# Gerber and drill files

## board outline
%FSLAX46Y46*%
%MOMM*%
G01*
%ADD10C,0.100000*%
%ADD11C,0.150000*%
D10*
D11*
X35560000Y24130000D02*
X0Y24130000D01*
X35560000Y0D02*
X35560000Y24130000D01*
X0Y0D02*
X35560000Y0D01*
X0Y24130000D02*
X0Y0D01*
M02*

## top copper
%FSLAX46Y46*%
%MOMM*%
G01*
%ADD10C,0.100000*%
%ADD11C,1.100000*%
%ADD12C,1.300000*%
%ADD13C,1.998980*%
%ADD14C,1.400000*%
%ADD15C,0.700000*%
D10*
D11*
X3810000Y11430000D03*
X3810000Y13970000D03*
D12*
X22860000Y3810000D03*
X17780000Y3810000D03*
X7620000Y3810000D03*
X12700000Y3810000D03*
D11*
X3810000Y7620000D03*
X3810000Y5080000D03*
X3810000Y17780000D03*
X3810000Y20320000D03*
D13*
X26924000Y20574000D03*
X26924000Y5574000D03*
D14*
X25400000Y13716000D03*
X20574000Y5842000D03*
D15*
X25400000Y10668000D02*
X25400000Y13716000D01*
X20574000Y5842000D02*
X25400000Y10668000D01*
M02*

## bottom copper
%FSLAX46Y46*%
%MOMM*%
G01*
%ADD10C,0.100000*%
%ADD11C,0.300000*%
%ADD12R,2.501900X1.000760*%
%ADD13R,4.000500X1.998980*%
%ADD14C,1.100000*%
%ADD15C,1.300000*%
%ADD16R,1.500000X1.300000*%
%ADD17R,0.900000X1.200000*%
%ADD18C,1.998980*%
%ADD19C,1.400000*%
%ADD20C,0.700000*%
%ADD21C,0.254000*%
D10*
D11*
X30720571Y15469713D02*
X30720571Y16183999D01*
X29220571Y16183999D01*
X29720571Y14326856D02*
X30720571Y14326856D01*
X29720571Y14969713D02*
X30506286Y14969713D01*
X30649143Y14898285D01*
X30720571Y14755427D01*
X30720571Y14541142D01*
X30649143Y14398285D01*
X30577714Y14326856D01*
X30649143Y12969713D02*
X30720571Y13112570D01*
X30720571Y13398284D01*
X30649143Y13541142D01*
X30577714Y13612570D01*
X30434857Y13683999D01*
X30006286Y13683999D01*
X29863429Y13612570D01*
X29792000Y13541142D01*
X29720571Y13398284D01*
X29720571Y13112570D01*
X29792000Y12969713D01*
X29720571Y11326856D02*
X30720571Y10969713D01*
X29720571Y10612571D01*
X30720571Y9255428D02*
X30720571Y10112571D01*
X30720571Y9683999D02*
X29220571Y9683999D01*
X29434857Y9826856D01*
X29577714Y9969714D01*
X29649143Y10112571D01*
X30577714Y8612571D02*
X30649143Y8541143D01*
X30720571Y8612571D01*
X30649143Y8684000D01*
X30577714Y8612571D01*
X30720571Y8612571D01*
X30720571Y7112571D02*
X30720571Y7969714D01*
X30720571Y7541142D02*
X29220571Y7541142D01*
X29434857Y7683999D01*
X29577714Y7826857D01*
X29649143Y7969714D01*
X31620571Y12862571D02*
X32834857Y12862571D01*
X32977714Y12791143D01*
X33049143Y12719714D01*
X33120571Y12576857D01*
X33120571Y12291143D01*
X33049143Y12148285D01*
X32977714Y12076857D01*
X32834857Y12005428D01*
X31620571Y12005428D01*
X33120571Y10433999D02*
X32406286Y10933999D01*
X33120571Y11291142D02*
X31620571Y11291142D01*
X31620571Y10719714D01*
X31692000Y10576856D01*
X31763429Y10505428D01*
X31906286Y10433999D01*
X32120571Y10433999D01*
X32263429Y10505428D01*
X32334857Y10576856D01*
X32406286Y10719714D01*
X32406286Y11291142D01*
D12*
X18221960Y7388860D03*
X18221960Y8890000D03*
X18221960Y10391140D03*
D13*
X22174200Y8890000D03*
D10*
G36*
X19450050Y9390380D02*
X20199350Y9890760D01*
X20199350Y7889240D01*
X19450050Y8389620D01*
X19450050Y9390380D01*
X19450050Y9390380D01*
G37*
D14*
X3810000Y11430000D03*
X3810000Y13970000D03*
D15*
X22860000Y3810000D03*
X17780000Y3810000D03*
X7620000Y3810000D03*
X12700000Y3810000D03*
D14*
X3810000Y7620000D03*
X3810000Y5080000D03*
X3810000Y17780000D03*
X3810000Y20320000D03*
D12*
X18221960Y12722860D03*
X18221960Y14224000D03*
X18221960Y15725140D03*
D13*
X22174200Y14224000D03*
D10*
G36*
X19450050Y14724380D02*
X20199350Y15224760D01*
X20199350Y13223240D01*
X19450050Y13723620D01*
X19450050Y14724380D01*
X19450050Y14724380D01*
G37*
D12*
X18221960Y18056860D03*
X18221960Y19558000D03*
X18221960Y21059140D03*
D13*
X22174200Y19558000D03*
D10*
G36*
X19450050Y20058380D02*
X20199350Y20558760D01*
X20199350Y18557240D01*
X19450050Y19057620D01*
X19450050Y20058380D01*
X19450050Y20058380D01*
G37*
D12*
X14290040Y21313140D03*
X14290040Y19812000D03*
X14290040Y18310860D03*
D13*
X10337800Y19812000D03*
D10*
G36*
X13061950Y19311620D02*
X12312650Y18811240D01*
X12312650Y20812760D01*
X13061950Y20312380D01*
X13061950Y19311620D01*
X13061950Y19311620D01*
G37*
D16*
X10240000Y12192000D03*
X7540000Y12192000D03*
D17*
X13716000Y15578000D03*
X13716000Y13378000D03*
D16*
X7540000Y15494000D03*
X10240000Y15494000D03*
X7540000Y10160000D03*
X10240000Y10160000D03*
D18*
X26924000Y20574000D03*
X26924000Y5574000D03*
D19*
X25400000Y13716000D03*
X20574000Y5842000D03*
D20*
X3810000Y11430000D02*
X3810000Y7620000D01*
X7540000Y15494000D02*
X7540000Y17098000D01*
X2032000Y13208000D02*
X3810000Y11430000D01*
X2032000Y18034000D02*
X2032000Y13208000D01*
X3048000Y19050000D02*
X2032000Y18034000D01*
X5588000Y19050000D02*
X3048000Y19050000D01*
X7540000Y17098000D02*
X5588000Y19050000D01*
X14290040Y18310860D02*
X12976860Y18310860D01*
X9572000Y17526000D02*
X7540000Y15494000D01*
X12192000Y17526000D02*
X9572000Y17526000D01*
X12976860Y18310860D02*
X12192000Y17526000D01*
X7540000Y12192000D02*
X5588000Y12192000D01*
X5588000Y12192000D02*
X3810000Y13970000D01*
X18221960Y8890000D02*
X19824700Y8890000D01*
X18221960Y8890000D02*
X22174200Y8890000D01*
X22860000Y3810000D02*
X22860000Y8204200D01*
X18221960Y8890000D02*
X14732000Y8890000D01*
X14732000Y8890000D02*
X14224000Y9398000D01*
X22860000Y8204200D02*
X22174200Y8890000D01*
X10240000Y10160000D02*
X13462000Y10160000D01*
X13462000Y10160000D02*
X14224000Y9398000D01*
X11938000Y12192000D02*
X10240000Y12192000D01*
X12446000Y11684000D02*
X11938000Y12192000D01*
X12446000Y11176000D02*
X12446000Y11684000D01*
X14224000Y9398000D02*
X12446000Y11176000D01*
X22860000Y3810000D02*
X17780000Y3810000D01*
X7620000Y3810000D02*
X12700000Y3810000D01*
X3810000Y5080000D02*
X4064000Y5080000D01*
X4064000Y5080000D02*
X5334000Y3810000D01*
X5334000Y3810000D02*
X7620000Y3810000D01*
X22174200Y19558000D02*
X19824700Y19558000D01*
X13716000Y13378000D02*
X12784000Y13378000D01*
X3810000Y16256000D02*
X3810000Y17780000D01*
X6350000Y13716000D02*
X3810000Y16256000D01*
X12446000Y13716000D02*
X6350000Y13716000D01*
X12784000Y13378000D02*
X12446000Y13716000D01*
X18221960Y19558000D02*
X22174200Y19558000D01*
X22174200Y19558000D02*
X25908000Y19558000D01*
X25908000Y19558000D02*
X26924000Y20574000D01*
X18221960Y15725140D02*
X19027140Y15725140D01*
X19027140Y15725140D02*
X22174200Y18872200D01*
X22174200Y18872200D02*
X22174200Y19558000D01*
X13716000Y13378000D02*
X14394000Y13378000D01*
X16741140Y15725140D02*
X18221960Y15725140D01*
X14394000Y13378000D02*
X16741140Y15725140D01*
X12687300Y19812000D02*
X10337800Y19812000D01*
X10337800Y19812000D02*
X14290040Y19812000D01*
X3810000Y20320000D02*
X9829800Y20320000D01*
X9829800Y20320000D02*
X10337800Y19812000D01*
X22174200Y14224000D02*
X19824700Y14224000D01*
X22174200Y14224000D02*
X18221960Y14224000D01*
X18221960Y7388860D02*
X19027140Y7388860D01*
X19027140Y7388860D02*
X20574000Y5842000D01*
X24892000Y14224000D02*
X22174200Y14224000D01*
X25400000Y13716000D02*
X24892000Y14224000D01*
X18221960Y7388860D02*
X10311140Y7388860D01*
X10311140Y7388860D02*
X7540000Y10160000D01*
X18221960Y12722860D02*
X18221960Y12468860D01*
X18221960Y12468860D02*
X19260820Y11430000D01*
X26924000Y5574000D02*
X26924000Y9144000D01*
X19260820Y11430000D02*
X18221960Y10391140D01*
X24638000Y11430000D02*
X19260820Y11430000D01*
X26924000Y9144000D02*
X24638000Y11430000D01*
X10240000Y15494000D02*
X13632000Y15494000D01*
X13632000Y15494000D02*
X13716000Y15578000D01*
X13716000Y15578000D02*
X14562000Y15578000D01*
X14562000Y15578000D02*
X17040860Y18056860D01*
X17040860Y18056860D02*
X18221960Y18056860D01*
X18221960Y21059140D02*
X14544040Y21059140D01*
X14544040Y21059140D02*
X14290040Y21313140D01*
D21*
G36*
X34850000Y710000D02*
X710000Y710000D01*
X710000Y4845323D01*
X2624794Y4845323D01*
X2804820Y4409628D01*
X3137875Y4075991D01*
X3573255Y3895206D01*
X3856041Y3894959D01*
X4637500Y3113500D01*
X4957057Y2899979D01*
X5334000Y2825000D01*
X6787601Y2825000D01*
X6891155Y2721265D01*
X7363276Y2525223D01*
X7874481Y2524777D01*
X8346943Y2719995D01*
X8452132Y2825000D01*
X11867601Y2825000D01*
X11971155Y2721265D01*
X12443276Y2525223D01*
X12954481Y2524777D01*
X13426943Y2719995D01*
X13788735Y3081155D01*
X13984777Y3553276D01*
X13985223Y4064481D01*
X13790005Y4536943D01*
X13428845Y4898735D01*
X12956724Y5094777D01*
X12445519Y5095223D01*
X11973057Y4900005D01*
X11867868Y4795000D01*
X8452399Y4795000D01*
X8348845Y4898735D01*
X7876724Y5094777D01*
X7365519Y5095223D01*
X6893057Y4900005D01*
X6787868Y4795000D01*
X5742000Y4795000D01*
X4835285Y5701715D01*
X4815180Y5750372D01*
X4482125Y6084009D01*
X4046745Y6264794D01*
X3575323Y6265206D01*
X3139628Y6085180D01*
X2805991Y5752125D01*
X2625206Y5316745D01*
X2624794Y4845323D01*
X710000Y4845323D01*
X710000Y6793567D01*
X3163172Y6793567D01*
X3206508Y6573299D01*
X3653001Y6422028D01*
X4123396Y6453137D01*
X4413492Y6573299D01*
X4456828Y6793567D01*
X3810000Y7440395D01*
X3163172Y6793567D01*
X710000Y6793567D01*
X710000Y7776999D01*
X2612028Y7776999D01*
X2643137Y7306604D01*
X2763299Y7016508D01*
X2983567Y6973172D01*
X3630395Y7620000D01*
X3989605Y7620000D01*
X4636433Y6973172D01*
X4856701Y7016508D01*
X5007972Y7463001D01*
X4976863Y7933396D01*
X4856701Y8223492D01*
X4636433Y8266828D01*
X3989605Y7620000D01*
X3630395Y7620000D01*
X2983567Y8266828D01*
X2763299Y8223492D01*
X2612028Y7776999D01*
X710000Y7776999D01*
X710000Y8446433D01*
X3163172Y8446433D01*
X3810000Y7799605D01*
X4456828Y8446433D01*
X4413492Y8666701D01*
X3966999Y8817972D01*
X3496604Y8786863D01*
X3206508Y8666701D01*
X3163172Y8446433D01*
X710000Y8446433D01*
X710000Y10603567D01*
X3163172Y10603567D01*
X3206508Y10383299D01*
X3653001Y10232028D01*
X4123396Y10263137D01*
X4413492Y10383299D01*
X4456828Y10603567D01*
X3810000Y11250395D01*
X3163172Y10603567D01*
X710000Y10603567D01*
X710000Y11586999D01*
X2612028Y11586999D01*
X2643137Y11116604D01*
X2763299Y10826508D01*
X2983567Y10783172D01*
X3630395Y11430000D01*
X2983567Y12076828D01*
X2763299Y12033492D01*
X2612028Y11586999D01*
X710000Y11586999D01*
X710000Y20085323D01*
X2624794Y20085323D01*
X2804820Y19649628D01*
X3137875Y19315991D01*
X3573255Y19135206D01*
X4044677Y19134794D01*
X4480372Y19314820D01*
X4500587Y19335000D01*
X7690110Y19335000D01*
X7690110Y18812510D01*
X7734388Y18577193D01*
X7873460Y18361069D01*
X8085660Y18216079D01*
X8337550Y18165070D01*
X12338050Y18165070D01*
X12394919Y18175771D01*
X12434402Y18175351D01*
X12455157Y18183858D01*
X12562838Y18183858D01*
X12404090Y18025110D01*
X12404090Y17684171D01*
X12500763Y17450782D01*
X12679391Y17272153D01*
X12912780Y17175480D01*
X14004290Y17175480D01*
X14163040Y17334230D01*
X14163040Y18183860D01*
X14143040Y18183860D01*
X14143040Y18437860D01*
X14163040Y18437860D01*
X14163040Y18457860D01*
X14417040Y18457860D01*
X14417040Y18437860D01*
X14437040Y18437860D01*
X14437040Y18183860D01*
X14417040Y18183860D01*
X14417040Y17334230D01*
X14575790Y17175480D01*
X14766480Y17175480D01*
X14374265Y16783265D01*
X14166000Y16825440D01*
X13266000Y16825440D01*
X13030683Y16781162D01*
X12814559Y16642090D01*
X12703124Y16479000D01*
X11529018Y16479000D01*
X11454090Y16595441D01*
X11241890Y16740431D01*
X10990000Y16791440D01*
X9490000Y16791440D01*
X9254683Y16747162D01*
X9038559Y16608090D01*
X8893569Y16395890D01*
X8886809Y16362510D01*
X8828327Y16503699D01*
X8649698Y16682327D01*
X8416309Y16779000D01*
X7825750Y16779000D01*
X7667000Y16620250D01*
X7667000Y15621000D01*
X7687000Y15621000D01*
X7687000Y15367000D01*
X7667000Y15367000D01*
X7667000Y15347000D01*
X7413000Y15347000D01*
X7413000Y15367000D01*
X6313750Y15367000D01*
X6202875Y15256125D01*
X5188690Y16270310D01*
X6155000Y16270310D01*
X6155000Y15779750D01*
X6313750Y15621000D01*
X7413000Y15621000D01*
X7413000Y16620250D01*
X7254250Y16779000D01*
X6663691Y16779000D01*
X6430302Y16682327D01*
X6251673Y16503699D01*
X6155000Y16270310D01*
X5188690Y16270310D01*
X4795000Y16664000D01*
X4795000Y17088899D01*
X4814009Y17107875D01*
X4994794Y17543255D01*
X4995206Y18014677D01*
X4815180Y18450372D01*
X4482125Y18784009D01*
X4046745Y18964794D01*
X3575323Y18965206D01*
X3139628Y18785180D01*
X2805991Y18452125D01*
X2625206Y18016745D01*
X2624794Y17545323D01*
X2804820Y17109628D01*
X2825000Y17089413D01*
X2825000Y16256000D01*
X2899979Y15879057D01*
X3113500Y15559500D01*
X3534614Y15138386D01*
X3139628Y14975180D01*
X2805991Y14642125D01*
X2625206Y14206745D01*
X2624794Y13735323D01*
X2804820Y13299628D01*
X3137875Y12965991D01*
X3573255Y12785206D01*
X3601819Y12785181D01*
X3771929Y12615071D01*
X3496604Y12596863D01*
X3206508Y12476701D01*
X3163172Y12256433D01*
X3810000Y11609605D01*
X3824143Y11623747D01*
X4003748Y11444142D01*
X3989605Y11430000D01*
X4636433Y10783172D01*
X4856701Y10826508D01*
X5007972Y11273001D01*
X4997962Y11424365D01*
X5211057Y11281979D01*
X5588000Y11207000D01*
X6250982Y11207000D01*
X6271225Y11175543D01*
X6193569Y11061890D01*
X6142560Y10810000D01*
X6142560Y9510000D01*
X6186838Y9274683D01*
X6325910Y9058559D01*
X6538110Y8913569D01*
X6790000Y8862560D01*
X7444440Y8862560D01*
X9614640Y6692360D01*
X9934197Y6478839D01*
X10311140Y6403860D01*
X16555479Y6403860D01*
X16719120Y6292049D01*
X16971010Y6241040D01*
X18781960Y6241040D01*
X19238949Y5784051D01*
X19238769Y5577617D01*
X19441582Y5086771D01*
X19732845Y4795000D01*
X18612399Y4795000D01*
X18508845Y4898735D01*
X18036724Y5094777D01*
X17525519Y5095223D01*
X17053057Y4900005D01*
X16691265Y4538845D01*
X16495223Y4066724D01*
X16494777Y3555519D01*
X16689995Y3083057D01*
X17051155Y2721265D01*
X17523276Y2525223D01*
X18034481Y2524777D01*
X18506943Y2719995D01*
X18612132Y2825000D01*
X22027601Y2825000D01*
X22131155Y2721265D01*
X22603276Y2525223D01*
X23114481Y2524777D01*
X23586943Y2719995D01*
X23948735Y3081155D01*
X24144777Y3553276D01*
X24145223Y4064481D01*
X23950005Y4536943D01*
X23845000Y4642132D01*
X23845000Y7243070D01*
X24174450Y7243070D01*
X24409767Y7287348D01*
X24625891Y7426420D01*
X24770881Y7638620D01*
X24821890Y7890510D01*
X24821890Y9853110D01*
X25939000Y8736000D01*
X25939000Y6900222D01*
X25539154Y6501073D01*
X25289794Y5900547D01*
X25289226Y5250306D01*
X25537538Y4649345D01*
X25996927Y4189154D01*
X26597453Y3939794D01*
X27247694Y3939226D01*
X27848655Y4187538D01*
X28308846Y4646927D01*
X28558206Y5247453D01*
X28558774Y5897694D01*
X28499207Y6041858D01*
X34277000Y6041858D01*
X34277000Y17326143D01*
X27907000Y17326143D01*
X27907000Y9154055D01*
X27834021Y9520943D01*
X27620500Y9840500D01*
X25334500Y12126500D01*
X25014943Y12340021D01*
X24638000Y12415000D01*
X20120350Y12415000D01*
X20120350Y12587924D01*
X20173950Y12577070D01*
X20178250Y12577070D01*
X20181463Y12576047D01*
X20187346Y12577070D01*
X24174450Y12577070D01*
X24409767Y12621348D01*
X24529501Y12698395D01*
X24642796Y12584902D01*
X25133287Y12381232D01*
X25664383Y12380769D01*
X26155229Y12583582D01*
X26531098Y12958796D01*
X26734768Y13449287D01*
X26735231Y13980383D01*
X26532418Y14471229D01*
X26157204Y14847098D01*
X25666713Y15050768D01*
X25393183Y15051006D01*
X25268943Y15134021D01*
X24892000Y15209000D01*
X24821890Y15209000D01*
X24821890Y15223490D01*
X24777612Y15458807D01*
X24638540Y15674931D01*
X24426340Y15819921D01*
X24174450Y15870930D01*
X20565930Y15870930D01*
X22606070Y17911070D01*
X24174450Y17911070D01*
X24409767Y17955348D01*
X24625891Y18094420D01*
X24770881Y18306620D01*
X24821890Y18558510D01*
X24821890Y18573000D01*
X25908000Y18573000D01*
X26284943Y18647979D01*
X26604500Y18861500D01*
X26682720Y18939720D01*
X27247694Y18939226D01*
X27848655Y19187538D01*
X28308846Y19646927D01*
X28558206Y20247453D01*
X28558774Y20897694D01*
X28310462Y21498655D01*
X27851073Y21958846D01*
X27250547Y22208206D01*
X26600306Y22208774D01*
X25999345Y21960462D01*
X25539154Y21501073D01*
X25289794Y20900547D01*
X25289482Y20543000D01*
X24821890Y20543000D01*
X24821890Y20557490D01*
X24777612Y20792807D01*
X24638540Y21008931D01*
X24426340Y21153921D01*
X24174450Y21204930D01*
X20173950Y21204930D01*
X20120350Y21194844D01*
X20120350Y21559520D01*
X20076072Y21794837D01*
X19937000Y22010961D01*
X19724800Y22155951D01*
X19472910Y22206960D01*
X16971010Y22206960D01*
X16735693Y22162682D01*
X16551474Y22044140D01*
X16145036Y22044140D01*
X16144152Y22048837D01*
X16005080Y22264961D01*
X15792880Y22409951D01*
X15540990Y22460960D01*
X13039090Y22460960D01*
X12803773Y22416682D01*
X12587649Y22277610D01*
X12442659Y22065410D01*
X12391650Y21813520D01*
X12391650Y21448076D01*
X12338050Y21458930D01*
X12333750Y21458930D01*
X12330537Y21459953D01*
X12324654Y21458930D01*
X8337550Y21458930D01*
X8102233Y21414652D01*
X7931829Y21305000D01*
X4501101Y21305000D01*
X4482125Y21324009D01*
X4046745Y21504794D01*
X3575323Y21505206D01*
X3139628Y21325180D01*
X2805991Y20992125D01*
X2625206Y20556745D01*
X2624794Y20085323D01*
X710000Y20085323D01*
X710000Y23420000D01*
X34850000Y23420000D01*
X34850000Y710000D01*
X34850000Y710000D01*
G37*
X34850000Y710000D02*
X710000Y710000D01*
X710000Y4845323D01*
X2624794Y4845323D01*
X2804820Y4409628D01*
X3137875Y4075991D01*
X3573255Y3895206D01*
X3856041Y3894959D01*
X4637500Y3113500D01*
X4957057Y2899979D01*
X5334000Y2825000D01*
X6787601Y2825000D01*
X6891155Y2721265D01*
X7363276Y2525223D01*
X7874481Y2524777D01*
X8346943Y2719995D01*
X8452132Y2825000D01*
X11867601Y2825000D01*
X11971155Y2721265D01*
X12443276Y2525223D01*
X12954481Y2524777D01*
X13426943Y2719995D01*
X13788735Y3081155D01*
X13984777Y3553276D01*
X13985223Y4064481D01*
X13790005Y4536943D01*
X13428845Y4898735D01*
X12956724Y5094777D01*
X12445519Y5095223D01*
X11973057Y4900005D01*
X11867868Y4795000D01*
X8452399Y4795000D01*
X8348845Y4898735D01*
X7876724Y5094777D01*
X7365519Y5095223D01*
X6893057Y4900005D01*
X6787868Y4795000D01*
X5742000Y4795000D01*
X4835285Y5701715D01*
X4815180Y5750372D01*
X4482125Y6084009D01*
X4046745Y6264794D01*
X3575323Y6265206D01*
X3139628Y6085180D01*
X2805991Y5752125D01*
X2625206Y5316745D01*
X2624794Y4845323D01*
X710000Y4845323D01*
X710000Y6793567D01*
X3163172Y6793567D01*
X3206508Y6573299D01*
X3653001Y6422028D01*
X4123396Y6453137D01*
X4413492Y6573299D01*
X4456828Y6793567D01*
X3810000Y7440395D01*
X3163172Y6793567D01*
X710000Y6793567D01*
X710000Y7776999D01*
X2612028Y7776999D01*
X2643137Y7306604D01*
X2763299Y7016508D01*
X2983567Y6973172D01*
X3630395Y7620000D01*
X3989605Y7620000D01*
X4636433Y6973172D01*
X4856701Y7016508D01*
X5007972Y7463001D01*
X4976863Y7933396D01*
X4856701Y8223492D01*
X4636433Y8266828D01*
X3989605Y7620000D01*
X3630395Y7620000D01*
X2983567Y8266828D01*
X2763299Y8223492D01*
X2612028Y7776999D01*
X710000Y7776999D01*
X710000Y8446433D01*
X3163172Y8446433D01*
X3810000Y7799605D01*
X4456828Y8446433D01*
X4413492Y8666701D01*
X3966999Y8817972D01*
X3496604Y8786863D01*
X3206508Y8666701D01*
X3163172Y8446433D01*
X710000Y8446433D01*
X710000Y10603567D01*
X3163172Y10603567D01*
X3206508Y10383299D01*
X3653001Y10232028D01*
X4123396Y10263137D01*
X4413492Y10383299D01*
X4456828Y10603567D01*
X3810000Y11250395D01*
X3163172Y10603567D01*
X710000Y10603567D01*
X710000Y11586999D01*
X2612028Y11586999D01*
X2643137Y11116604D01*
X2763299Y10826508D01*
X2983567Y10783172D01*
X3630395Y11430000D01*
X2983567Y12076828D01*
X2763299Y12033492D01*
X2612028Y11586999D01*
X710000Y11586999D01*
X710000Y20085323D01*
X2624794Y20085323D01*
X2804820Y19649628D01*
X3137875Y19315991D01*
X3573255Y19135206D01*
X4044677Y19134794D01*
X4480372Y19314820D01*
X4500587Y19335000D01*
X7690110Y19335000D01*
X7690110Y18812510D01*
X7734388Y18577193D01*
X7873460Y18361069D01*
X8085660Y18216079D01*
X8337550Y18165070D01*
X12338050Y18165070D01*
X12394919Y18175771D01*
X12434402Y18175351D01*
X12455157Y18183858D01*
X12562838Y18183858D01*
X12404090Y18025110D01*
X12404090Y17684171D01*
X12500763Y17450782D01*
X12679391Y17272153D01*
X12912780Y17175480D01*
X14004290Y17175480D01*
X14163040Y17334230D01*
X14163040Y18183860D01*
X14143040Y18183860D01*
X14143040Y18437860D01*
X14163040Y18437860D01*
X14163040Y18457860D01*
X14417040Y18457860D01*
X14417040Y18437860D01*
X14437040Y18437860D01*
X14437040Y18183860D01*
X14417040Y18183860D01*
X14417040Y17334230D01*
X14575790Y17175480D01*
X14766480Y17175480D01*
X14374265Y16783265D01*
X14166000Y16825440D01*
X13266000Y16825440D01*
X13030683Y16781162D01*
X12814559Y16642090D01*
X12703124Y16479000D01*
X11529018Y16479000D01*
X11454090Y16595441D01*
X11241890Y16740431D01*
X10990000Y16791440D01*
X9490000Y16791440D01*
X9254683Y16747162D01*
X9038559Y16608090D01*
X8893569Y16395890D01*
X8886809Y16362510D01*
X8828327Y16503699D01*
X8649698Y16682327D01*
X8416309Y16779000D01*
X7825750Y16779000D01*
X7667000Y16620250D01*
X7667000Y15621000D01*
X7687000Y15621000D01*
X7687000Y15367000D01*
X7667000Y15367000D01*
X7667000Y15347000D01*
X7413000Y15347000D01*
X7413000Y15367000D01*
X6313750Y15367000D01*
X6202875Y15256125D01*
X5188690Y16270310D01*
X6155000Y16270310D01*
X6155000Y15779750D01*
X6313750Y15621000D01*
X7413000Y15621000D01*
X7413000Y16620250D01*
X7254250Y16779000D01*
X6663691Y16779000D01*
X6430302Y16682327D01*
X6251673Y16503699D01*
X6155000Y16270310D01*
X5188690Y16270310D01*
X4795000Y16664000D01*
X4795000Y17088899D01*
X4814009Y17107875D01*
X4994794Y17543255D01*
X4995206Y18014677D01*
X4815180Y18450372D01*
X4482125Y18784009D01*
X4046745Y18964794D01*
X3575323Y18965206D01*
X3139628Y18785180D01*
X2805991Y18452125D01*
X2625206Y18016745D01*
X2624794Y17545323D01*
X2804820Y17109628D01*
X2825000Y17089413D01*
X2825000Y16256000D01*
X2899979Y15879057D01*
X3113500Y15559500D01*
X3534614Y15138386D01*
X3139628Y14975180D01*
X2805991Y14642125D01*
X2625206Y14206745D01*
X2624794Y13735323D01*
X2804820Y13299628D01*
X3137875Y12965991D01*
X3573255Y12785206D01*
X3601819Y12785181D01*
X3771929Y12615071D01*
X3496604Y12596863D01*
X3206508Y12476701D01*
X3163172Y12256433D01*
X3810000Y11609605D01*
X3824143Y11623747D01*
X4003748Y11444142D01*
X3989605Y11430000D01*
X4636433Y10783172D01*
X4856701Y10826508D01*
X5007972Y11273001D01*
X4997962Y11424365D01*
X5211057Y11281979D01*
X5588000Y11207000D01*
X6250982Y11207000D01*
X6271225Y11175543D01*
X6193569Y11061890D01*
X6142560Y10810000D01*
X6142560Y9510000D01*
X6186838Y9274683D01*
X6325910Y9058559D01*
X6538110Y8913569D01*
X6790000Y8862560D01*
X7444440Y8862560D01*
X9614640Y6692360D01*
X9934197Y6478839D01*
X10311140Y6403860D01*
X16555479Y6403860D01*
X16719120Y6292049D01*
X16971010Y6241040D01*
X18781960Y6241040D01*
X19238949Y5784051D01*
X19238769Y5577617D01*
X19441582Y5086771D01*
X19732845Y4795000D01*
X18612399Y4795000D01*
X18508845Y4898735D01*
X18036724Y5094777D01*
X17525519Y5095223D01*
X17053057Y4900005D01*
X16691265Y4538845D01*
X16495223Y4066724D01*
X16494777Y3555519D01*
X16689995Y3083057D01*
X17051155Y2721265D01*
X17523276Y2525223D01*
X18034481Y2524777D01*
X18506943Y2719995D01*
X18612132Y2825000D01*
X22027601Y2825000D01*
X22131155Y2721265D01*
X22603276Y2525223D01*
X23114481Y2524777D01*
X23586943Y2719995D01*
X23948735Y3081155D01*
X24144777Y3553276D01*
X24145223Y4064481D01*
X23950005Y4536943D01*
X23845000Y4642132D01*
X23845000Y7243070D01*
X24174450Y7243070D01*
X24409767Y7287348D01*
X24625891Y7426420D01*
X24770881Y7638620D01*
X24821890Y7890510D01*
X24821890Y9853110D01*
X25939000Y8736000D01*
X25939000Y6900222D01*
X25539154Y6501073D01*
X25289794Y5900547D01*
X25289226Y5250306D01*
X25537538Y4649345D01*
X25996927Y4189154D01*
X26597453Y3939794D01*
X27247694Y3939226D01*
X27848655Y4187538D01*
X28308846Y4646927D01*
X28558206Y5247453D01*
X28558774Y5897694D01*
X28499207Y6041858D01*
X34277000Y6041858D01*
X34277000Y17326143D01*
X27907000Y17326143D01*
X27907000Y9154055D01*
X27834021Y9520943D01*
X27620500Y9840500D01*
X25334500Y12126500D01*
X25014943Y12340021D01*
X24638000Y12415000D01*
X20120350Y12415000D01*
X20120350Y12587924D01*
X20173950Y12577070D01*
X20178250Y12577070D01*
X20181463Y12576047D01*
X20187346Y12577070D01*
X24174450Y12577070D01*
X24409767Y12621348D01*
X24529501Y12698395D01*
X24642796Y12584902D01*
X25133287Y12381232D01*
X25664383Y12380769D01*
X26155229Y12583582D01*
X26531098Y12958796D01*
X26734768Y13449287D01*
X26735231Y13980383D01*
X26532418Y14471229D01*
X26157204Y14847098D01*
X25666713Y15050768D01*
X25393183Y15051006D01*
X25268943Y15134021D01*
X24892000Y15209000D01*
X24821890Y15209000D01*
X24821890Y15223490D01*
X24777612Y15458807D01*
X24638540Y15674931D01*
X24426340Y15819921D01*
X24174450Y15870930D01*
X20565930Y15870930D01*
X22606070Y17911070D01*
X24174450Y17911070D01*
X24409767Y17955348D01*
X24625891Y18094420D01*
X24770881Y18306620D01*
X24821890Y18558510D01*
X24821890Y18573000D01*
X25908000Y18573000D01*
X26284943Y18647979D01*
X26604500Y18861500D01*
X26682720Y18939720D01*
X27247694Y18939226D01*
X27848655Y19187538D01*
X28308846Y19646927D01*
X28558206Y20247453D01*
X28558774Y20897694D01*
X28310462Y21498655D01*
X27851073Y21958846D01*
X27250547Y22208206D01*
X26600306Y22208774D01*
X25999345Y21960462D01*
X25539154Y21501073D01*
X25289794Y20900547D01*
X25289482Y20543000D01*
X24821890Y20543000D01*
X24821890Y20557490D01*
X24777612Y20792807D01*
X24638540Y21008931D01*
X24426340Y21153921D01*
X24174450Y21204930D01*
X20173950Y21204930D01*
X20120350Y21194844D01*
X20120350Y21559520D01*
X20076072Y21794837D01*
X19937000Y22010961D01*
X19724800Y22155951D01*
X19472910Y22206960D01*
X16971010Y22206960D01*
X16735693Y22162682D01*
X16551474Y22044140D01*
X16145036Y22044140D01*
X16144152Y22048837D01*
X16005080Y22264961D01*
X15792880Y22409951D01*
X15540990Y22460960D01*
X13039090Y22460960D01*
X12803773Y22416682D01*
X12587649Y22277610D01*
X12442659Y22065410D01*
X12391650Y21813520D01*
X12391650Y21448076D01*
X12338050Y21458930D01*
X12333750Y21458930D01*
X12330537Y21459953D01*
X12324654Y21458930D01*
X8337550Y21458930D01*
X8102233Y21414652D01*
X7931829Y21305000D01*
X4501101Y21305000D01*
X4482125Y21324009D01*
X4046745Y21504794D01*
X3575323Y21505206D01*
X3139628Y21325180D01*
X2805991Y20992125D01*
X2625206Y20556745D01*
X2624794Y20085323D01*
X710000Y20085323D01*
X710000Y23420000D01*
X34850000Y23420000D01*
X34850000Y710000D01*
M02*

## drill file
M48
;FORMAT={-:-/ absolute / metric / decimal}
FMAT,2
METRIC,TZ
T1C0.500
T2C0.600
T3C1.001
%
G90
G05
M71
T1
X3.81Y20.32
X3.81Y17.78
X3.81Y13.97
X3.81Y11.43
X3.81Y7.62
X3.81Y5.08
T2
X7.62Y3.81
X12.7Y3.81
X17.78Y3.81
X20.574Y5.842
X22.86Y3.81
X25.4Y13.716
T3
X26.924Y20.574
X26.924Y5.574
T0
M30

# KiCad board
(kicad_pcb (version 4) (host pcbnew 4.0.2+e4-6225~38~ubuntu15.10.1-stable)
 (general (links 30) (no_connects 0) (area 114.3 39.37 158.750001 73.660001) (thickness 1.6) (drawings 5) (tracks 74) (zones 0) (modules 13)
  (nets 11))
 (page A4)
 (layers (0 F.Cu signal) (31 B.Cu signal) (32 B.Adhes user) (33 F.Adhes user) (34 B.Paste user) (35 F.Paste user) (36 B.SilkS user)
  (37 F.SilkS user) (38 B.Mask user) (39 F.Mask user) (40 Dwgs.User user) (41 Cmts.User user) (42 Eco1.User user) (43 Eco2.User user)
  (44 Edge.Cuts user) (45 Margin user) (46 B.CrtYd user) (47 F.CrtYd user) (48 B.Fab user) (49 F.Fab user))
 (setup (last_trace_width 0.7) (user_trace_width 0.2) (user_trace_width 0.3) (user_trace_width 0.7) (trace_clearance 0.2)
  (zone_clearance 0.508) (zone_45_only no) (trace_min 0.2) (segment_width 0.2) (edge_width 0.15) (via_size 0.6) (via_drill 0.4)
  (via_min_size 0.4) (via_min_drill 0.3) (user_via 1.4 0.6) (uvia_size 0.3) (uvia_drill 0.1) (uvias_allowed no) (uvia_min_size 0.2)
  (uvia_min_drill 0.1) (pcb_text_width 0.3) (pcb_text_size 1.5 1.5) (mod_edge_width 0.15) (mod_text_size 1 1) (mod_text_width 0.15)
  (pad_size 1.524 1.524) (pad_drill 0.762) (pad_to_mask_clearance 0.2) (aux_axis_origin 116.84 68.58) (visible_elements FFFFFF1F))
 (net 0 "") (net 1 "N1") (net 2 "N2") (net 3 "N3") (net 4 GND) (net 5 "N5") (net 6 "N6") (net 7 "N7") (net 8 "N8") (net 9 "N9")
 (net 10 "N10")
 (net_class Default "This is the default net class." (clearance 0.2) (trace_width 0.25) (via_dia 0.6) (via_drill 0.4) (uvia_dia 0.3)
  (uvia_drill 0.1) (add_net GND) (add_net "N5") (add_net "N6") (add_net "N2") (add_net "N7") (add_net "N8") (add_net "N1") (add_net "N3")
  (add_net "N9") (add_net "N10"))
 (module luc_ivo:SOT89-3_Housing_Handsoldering (layer B.Cu) (at 137.414 59.69 90)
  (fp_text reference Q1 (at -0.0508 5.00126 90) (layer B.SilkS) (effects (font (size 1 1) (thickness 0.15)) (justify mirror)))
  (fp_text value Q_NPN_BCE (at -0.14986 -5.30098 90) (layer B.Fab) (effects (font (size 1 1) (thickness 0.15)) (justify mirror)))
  (pad 1 smd rect (at -1.50114 -2.35204 90) (size 1.00076 2.5019) (layers B.Cu B.Paste B.Mask) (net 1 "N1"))
  (pad 2 smd rect (at 0 -2.35204 90) (size 1.00076 2.5019) (layers B.Cu B.Paste B.Mask) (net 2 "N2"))
  (pad 3 smd rect (at 1.50114 -2.35204 90) (size 1.00076 2.5019) (layers B.Cu B.Paste B.Mask) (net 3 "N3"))
  (pad 2 smd rect (at 0 1.6002 90) (size 1.99898 4.0005) (layers B.Cu B.Paste B.Mask) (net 2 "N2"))
  (pad 2 smd trapezoid (at 0 -0.7493 270) (size 1.50114 0.7493) (rect_delta 0 -0.50038) (layers B.Cu B.Paste B.Mask) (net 2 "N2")))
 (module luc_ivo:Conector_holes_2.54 (layer F.Cu) (at 120.65 55.88 90)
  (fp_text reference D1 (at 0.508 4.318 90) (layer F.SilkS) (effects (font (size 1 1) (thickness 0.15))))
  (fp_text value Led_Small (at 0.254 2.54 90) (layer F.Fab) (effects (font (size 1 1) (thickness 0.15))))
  (pad 1 thru_hole circle (at -1.27 0 90) (size 1.1 1.1) (drill 0.5) (layers *.Cu *.Mask F.SilkS) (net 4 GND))
  (pad 2 thru_hole circle (at 1.27 0 90) (size 1.1 1.1) (drill 0.5) (layers *.Cu *.Mask F.SilkS) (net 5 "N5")))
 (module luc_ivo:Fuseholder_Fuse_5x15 (layer F.Cu) (at 132.08 64.77)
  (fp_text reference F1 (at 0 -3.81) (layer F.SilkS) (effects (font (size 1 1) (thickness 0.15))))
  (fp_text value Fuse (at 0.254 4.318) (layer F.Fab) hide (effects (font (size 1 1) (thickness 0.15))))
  (pad 2 thru_hole circle (at 7.62 0) (size 1.3 1.3) (drill 0.6) (layers *.Cu *.Mask) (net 2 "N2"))
  (pad 2 thru_hole circle (at 2.54 0) (size 1.3 1.3) (drill 0.6) (layers *.Cu *.Mask) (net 2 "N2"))
  (pad 1 thru_hole circle (at -7.62 0) (size 1.3 1.3) (drill 0.6) (layers *.Cu *.Mask) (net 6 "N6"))
  (pad 1 thru_hole circle (at -2.54 0) (size 1.3 1.3) (drill 0.6) (layers *.Cu *.Mask) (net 6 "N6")))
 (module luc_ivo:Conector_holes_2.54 (layer F.Cu) (at 120.65 62.23 270)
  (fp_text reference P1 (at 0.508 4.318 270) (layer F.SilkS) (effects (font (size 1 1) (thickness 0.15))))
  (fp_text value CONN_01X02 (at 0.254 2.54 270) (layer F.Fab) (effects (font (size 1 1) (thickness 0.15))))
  (pad 1 thru_hole circle (at -1.27 0 270) (size 1.1 1.1) (drill 0.5) (layers *.Cu *.Mask F.SilkS) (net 4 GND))
  (pad 2 thru_hole circle (at 1.27 0 270) (size 1.1 1.1) (drill 0.5) (layers *.Cu *.Mask F.SilkS) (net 6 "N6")))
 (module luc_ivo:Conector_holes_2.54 (layer F.Cu) (at 120.65 49.53 90)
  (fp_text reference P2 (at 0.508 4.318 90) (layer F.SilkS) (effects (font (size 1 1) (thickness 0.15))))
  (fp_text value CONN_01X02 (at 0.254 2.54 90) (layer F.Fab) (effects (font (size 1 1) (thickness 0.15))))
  (pad 1 thru_hole circle (at -1.27 0 90) (size 1.1 1.1) (drill 0.5) (layers *.Cu *.Mask F.SilkS) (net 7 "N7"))
  (pad 2 thru_hole circle (at 1.27 0 90) (size 1.1 1.1) (drill 0.5) (layers *.Cu *.Mask F.SilkS) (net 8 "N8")))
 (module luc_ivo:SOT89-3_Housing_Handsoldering (layer B.Cu) (at 137.414 54.356 90)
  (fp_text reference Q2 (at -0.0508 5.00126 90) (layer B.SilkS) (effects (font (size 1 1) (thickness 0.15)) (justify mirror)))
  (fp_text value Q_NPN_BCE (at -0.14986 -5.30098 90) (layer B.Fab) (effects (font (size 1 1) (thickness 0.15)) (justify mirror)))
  (pad 1 smd rect (at -1.50114 -2.35204 90) (size 1.00076 2.5019) (layers B.Cu B.Paste B.Mask) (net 3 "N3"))
  (pad 2 smd rect (at 0 -2.35204 90) (size 1.00076 2.5019) (layers B.Cu B.Paste B.Mask) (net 1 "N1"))
  (pad 3 smd rect (at 1.50114 -2.35204 90) (size 1.00076 2.5019) (layers B.Cu B.Paste B.Mask) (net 7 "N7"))
  (pad 2 smd rect (at 0 1.6002 90) (size 1.99898 4.0005) (layers B.Cu B.Paste B.Mask) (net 1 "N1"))
  (pad 2 smd trapezoid (at 0 -0.7493 270) (size 1.50114 0.7493) (rect_delta 0 -0.50038) (layers B.Cu B.Paste B.Mask) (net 1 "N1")))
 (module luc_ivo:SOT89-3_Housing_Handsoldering (layer B.Cu) (at 137.414 49.022 90)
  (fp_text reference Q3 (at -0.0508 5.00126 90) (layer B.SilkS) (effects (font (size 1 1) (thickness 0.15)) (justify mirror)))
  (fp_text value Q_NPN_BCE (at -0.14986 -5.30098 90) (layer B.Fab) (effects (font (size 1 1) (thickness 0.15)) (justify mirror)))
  (pad 1 smd rect (at -1.50114 -2.35204 90) (size 1.00076 2.5019) (layers B.Cu B.Paste B.Mask) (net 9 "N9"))
  (pad 2 smd rect (at 0 -2.35204 90) (size 1.00076 2.5019) (layers B.Cu B.Paste B.Mask) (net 7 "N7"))
  (pad 3 smd rect (at 1.50114 -2.35204 90) (size 1.00076 2.5019) (layers B.Cu B.Paste B.Mask) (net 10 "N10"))
  (pad 2 smd rect (at 0 1.6002 90) (size 1.99898 4.0005) (layers B.Cu B.Paste B.Mask) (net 7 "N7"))
  (pad 2 smd trapezoid (at 0 -0.7493 270) (size 1.50114 0.7493) (rect_delta 0 -0.50038) (layers B.Cu B.Paste B.Mask) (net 7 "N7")))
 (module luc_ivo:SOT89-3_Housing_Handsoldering (layer B.Cu) (at 128.778 48.768 270)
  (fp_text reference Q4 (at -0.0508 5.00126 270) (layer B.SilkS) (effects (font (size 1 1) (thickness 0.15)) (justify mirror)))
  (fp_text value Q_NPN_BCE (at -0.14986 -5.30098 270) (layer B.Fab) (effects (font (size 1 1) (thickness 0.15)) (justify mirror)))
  (pad 1 smd rect (at -1.50114 -2.35204 270) (size 1.00076 2.5019) (layers B.Cu B.Paste B.Mask) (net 10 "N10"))
  (pad 2 smd rect (at 0 -2.35204 270) (size 1.00076 2.5019) (layers B.Cu B.Paste B.Mask) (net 8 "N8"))
  (pad 3 smd rect (at 1.50114 -2.35204 270) (size 1.00076 2.5019) (layers B.Cu B.Paste B.Mask) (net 4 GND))
  (pad 2 smd rect (at 0 1.6002 270) (size 1.99898 4.0005) (layers B.Cu B.Paste B.Mask) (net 8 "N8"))
  (pad 2 smd trapezoid (at 0 -0.7493 90) (size 1.50114 0.7493) (rect_delta 0 -0.50038) (layers B.Cu B.Paste B.Mask) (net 8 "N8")))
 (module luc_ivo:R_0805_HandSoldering (layer B.Cu) (at 125.73 56.388 180)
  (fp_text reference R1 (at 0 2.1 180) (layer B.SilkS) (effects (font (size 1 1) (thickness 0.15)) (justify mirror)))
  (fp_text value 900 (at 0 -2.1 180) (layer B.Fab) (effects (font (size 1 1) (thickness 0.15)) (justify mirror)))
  (pad 1 smd rect (at -1.35 0 180) (size 1.5 1.3) (layers B.Cu B.Paste B.Mask) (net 2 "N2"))
  (pad 2 smd rect (at 1.35 0 180) (size 1.5 1.3) (layers B.Cu B.Paste B.Mask) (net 5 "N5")))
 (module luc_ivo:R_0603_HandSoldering (layer B.Cu) (at 130.556 54.102 270)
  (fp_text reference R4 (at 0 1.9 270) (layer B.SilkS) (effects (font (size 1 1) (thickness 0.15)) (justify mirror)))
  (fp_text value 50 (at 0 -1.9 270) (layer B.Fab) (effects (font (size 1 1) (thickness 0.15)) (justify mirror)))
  (pad 1 smd rect (at -1.1 0 270) (size 1.2 0.9) (layers B.Cu B.Paste B.Mask) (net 9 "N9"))
  (pad 2 smd rect (at 1.1 0 270) (size 1.2 0.9) (layers B.Cu B.Paste B.Mask) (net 7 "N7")))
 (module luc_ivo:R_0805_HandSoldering (layer B.Cu) (at 125.73 53.086)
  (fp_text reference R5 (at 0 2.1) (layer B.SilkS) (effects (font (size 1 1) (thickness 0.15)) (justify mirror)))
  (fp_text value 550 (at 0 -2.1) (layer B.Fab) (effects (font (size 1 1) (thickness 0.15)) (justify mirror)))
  (pad 1 smd rect (at -1.35 0) (size 1.5 1.3) (layers B.Cu B.Paste B.Mask) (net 4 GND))
  (pad 2 smd rect (at 1.35 0) (size 1.5 1.3) (layers B.Cu B.Paste B.Mask) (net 9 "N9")))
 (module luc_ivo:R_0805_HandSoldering (layer B.Cu) (at 125.73 58.42)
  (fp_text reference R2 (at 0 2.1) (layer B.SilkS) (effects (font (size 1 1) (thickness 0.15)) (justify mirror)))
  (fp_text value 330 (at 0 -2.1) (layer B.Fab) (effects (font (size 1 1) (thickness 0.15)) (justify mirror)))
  (pad 1 smd rect (at -1.35 0) (size 1.5 1.3) (layers B.Cu B.Paste B.Mask) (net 1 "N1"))
  (pad 2 smd rect (at 1.35 0) (size 1.5 1.3) (layers B.Cu B.Paste B.Mask) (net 2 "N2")))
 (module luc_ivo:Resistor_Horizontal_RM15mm (layer F.Cu) (at 143.764 48.006 270)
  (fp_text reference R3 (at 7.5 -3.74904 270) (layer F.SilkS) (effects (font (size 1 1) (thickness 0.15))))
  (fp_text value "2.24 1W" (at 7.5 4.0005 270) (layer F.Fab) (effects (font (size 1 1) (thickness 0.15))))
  (pad 1 thru_hole circle (at 0 0 270) (size 1.99898 1.99898) (drill 1.00076) (layers *.Cu *.SilkS *.Mask) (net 7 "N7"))
  (pad 2 thru_hole circle (at 15 0 270) (size 1.99898 1.99898) (drill 1.00076) (layers *.Cu *.SilkS *.Mask) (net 3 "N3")))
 (gr_line (start 152.4 44.45) (end 116.84 44.45) (angle 90) (layer Edge.Cuts) (width 0.15))
 (gr_line (start 152.4 68.58) (end 152.4 44.45) (angle 90) (layer Edge.Cuts) (width 0.15))
 (gr_line (start 116.84 68.58) (end 152.4 68.58) (angle 90) (layer Edge.Cuts) (width 0.15))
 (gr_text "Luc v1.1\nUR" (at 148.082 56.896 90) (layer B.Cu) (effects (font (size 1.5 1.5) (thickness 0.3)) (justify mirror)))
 (gr_line (start 116.84 44.45) (end 116.84 68.58) (angle 90) (layer Edge.Cuts) (width 0.15))
 (segment (start 120.65 57.15) (end 120.65 60.96) (width 0.7) (layer B.Cu) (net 4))
 (segment (start 124.38 53.086) (end 124.38 51.482) (width 0.7) (layer B.Cu) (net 4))
 (segment (start 118.872 55.372) (end 120.65 57.15) (width 0.7) (layer B.Cu) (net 4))
 (segment (start 118.872 50.546) (end 118.872 55.372) (width 0.7) (layer B.Cu) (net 4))
 (segment (start 119.888 49.53) (end 118.872 50.546) (width 0.7) (layer B.Cu) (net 4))
 (segment (start 122.428 49.53) (end 119.888 49.53) (width 0.7) (layer B.Cu) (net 4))
 (segment (start 124.38 51.482) (end 122.428 49.53) (width 0.7) (layer B.Cu) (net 4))
 (segment (start 131.13004 50.26914) (end 129.81686 50.26914) (width 0.7) (layer B.Cu) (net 4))
 (segment (start 126.412 51.054) (end 124.38 53.086) (width 0.7) (layer B.Cu) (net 4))
 (segment (start 129.032 51.054) (end 126.412 51.054) (width 0.7) (layer B.Cu) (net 4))
 (segment (start 129.81686 50.26914) (end 129.032 51.054) (width 0.7) (layer B.Cu) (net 4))
 (segment (start 124.38 56.388) (end 122.428 56.388) (width 0.7) (layer B.Cu) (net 5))
 (segment (start 122.428 56.388) (end 120.65 54.61) (width 0.7) (layer B.Cu) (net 5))
 (segment (start 135.06196 59.69) (end 136.6647 59.69) (width 0.7) (layer B.Cu) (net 2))
 (segment (start 135.06196 59.69) (end 139.0142 59.69) (width 0.7) (layer B.Cu) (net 2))
 (segment (start 139.7 64.77) (end 139.7 60.3758) (width 0.7) (layer B.Cu) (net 2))
 (segment (start 135.06196 59.69) (end 131.572 59.69) (width 0.7) (layer B.Cu) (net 2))
 (segment (start 131.572 59.69) (end 131.064 59.182) (width 0.7) (layer B.Cu) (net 2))
 (segment (start 139.7 60.3758) (end 139.0142 59.69) (width 0.7) (layer B.Cu) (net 2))
 (segment (start 127.08 58.42) (end 130.302 58.42) (width 0.7) (layer B.Cu) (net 2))
 (segment (start 130.302 58.42) (end 131.064 59.182) (width 0.7) (layer B.Cu) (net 2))
 (segment (start 128.778 56.388) (end 127.08 56.388) (width 0.7) (layer B.Cu) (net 2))
 (segment (start 129.286 56.896) (end 128.778 56.388) (width 0.7) (layer B.Cu) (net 2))
 (segment (start 129.286 57.404) (end 129.286 56.896) (width 0.7) (layer B.Cu) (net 2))
 (segment (start 131.064 59.182) (end 129.286 57.404) (width 0.7) (layer B.Cu) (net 2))
 (segment (start 139.7 64.77) (end 134.62 64.77) (width 0.7) (layer B.Cu) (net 2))
 (segment (start 124.46 64.77) (end 129.54 64.77) (width 0.7) (layer B.Cu) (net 6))
 (segment (start 120.65 63.5) (end 120.904 63.5) (width 0.7) (layer B.Cu) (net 6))
 (segment (start 120.904 63.5) (end 122.174 64.77) (width 0.7) (layer B.Cu) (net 6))
 (segment (start 122.174 64.77) (end 124.46 64.77) (width 0.7) (layer B.Cu) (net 6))
 (segment (start 139.0142 49.022) (end 136.6647 49.022) (width 0.7) (layer B.Cu) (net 7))
 (segment (start 130.556 55.202) (end 129.624 55.202) (width 0.7) (layer B.Cu) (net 7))
 (segment (start 120.65 52.324) (end 120.65 50.8) (width 0.7) (layer B.Cu) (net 7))
 (segment (start 123.19 54.864) (end 120.65 52.324) (width 0.7) (layer B.Cu) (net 7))
 (segment (start 129.286 54.864) (end 123.19 54.864) (width 0.7) (layer B.Cu) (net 7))
 (segment (start 129.624 55.202) (end 129.286 54.864) (width 0.7) (layer B.Cu) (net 7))
 (segment (start 135.06196 49.022) (end 139.0142 49.022) (width 0.7) (layer B.Cu) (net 7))
 (segment (start 139.0142 49.022) (end 142.748 49.022) (width 0.7) (layer B.Cu) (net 7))
 (segment (start 142.748 49.022) (end 143.764 48.006) (width 0.7) (layer B.Cu) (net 7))
 (segment (start 135.06196 52.85486) (end 135.86714 52.85486) (width 0.7) (layer B.Cu) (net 7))
 (segment (start 135.86714 52.85486) (end 139.0142 49.7078) (width 0.7) (layer B.Cu) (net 7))
 (segment (start 139.0142 49.7078) (end 139.0142 49.022) (width 0.7) (layer B.Cu) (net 7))
 (segment (start 130.556 55.202) (end 131.234 55.202) (width 0.7) (layer B.Cu) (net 7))
 (segment (start 133.58114 52.85486) (end 135.06196 52.85486) (width 0.7) (layer B.Cu) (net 7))
 (segment (start 131.234 55.202) (end 133.58114 52.85486) (width 0.7) (layer B.Cu) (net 7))
 (segment (start 129.5273 48.768) (end 127.1778 48.768) (width 0.7) (layer B.Cu) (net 8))
 (segment (start 127.1778 48.768) (end 131.13004 48.768) (width 0.7) (layer B.Cu) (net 8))
 (segment (start 120.65 48.26) (end 126.6698 48.26) (width 0.7) (layer B.Cu) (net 8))
 (segment (start 126.6698 48.26) (end 127.1778 48.768) (width 0.7) (layer B.Cu) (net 8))
 (segment (start 139.0142 54.356) (end 136.6647 54.356) (width 0.7) (layer B.Cu) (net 1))
 (segment (start 139.0142 54.356) (end 135.06196 54.356) (width 0.7) (layer B.Cu) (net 1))
 (segment (start 135.06196 61.19114) (end 135.86714 61.19114) (width 0.7) (layer B.Cu) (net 1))
 (segment (start 135.86714 61.19114) (end 137.414 62.738) (width 0.7) (layer B.Cu) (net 1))
 (segment (start 141.732 54.356) (end 139.0142 54.356) (width 0.7) (layer B.Cu) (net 1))
 (segment (start 142.24 54.864) (end 141.732 54.356) (width 0.7) (layer B.Cu) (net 1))
 (via (at 142.24 54.864) (size 1.4) (drill 0.6) (layers F.Cu B.Cu) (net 1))
 (segment (start 142.24 57.912) (end 142.24 54.864) (width 0.7) (layer F.Cu) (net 1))
 (segment (start 137.414 62.738) (end 142.24 57.912) (width 0.7) (layer F.Cu) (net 1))
 (via (at 137.414 62.738) (size 1.4) (drill 0.6) (layers F.Cu B.Cu) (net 1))
 (segment (start 135.06196 61.19114) (end 127.15114 61.19114) (width 0.7) (layer B.Cu) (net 1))
 (segment (start 127.15114 61.19114) (end 124.38 58.42) (width 0.7) (layer B.Cu) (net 1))
 (segment (start 135.06196 55.85714) (end 135.06196 56.11114) (width 0.7) (layer B.Cu) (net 3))
 (segment (start 135.06196 56.11114) (end 136.10082 57.15) (width 0.7) (layer B.Cu) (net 3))
 (segment (start 143.764 63.006) (end 143.764 59.436) (width 0.7) (layer B.Cu) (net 3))
 (segment (start 136.10082 57.15) (end 135.06196 58.18886) (width 0.7) (layer B.Cu) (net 3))
 (segment (start 141.478 57.15) (end 136.10082 57.15) (width 0.7) (layer B.Cu) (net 3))
 (segment (start 143.764 59.436) (end 141.478 57.15) (width 0.7) (layer B.Cu) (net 3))
 (segment (start 127.08 53.086) (end 130.472 53.086) (width 0.7) (layer B.Cu) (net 9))
 (segment (start 130.472 53.086) (end 130.556 53.002) (width 0.7) (layer B.Cu) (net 9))
 (segment (start 130.556 53.002) (end 131.402 53.002) (width 0.7) (layer B.Cu) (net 9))
 (segment (start 131.402 53.002) (end 133.88086 50.52314) (width 0.7) (layer B.Cu) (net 9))
 (segment (start 133.88086 50.52314) (end 135.06196 50.52314) (width 0.7) (layer B.Cu) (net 9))
 (segment (start 135.06196 47.52086) (end 131.38404 47.52086) (width 0.7) (layer B.Cu) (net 10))
 (segment (start 131.38404 47.52086) (end 131.13004 47.26686) (width 0.7) (layer B.Cu) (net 10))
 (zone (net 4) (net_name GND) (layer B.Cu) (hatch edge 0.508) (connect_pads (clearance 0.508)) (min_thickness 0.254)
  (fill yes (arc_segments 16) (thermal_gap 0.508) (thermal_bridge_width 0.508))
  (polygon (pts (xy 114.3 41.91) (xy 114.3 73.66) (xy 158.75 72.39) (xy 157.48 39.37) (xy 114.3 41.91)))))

